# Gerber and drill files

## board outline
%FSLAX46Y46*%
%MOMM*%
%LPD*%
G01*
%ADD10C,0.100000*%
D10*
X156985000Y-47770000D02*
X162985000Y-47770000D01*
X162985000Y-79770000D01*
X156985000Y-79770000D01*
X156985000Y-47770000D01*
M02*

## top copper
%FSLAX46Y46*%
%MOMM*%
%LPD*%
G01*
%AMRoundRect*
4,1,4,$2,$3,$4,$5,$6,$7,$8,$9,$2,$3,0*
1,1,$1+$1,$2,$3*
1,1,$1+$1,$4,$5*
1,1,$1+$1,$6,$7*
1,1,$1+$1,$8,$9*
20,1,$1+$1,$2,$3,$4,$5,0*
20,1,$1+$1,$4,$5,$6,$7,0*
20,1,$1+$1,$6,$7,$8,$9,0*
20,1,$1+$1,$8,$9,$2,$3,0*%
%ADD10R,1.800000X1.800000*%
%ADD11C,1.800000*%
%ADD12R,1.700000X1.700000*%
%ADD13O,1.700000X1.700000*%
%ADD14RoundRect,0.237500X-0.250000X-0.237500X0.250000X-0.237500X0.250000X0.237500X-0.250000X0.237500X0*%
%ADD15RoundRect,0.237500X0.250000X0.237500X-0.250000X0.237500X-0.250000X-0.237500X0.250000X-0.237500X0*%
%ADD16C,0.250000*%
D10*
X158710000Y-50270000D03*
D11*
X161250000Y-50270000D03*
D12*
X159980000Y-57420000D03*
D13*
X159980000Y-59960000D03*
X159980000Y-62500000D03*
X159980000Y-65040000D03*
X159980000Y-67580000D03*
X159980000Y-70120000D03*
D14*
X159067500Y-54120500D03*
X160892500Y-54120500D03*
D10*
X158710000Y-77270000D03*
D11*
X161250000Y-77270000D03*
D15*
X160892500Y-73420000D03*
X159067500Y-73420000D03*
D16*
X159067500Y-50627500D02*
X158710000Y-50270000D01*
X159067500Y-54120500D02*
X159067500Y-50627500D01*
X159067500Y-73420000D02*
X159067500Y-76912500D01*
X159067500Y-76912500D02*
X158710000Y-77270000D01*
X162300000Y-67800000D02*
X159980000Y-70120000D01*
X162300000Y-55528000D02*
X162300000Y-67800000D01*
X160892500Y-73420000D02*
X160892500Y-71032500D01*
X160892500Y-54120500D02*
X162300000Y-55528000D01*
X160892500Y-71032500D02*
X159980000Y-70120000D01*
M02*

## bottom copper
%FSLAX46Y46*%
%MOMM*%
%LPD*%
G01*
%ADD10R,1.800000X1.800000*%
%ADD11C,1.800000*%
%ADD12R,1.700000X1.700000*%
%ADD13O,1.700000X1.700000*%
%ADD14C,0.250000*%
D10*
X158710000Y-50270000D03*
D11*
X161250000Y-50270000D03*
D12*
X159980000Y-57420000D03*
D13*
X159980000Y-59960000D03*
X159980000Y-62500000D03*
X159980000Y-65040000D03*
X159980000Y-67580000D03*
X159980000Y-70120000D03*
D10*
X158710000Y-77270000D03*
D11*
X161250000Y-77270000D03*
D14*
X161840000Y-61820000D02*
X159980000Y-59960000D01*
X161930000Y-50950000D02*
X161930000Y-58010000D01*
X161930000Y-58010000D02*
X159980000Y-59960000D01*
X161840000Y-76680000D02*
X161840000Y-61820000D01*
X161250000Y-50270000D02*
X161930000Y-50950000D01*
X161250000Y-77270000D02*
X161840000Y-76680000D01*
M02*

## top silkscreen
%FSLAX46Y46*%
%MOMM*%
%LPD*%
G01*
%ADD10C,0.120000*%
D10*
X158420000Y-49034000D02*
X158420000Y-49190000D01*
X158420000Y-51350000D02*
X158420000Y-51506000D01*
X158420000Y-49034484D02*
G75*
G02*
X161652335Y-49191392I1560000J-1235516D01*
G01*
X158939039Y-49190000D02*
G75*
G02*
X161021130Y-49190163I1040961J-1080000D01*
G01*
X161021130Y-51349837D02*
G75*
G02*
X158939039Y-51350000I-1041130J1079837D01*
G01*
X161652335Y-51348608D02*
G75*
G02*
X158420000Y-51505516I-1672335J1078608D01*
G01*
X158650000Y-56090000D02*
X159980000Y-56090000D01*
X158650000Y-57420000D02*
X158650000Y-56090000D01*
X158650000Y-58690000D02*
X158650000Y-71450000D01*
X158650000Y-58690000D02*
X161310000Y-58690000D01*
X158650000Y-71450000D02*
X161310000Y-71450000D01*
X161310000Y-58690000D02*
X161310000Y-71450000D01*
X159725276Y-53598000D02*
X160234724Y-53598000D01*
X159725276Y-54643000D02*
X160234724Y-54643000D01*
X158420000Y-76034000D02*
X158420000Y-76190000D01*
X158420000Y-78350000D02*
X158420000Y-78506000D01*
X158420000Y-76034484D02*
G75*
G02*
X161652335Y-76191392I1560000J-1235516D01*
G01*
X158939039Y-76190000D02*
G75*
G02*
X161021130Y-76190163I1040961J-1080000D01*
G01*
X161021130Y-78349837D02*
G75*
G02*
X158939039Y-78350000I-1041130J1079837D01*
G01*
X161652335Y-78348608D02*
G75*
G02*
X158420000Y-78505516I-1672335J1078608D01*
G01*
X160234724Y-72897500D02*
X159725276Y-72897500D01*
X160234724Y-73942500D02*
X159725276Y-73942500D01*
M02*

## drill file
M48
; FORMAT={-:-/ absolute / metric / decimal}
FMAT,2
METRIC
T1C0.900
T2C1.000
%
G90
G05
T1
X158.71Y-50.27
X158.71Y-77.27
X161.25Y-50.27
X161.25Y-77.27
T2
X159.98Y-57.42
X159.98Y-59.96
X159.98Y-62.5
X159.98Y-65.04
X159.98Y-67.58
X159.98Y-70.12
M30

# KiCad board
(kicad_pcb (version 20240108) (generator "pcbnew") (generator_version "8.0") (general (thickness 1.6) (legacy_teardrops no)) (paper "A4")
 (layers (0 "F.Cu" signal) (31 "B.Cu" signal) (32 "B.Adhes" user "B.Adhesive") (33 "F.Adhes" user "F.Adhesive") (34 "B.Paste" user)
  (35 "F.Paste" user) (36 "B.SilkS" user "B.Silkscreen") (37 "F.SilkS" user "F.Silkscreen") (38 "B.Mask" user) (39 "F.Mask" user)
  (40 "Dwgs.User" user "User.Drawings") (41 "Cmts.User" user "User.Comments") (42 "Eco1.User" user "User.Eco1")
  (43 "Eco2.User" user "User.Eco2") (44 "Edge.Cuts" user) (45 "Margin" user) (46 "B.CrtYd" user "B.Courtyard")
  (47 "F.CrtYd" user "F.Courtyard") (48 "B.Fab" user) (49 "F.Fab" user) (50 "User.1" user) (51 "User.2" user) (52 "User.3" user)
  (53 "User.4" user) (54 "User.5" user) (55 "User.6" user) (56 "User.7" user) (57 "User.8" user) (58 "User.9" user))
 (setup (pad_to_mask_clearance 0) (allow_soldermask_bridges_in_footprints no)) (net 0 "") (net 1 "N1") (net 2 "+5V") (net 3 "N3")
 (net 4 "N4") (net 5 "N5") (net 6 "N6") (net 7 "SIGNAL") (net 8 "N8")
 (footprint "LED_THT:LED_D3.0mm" (layer "F.Cu") (at 158.71 50.27)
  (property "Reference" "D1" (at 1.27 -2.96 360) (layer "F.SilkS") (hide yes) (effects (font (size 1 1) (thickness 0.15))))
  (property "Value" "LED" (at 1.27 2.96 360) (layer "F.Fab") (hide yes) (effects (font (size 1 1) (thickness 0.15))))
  (fp_line (start -0.29 -1.236) (end -0.29 -1.08) (stroke (width 0.12) (type solid)) (layer "F.SilkS"))
  (fp_line (start -0.29 1.08) (end -0.29 1.236) (stroke (width 0.12) (type solid)) (layer "F.SilkS"))
  (fp_arc (start -0.29 -1.235516) (mid 1.366487 -1.987659) (end 2.942335 -1.078608) (stroke (width 0.12) (type solid)) (layer "F.SilkS"))
  (fp_arc (start 0.229039 -1.08) (mid 1.270117 -1.5) (end 2.31113 -1.079837) (stroke (width 0.12) (type solid)) (layer "F.SilkS"))
  (fp_arc (start 2.31113 1.079837) (mid 1.270117 1.5) (end 0.229039 1.08) (stroke (width 0.12) (type solid)) (layer "F.SilkS"))
  (fp_arc (start 2.942335 1.078608) (mid 1.366487 1.987659) (end -0.29 1.235516) (stroke (width 0.12) (type solid)) (layer "F.SilkS"))
  (pad "1" thru_hole rect (at 0 0) (size 1.8 1.8) (drill 0.9) (layers "*.Cu" "*.Mask") (remove_unused_layers no) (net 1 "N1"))
  (pad "2" thru_hole circle (at 2.54 0) (size 1.8 1.8) (drill 0.9) (layers "*.Cu" "*.Mask") (remove_unused_layers no) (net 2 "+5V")))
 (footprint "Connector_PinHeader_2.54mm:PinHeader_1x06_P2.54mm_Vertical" (layer "F.Cu") (at 159.98 57.42)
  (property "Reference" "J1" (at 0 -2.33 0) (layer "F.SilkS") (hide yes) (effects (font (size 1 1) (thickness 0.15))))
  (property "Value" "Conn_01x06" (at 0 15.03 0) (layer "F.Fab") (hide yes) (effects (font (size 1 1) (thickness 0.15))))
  (fp_line (start -1.33 -1.33) (end 0 -1.33) (stroke (width 0.12) (type solid)) (layer "F.SilkS"))
  (fp_line (start -1.33 0) (end -1.33 -1.33) (stroke (width 0.12) (type solid)) (layer "F.SilkS"))
  (fp_line (start -1.33 1.27) (end -1.33 14.03) (stroke (width 0.12) (type solid)) (layer "F.SilkS"))
  (fp_line (start -1.33 1.27) (end 1.33 1.27) (stroke (width 0.12) (type solid)) (layer "F.SilkS"))
  (fp_line (start -1.33 14.03) (end 1.33 14.03) (stroke (width 0.12) (type solid)) (layer "F.SilkS"))
  (fp_line (start 1.33 1.27) (end 1.33 14.03) (stroke (width 0.12) (type solid)) (layer "F.SilkS"))
  (pad "1" thru_hole rect (at 0 0) (size 1.7 1.7) (drill 1) (layers "*.Cu" "*.Mask") (remove_unused_layers no) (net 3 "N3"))
  (pad "2" thru_hole oval (at 0 2.54) (size 1.7 1.7) (drill 1) (layers "*.Cu" "*.Mask") (remove_unused_layers no) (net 2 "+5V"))
  (pad "3" thru_hole oval (at 0 5.08) (size 1.7 1.7) (drill 1) (layers "*.Cu" "*.Mask") (remove_unused_layers no) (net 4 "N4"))
  (pad "4" thru_hole oval (at 0 7.62) (size 1.7 1.7) (drill 1) (layers "*.Cu" "*.Mask") (remove_unused_layers no) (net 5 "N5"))
  (pad "5" thru_hole oval (at 0 10.16) (size 1.7 1.7) (drill 1) (layers "*.Cu" "*.Mask") (remove_unused_layers no) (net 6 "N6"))
  (pad "6" thru_hole oval (at 0 12.7) (size 1.7 1.7) (drill 1) (layers "*.Cu" "*.Mask") (remove_unused_layers no) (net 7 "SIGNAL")))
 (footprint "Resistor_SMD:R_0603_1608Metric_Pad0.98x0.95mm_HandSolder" (layer "F.Cu") (at 159.98 54.1205)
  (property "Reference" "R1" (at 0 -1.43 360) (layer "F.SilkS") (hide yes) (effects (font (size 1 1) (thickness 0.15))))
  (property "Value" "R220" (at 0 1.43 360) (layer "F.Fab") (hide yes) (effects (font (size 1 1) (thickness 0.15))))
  (fp_line (start -0.254724 -0.5225) (end 0.254724 -0.5225) (stroke (width 0.12) (type solid)) (layer "F.SilkS"))
  (fp_line (start -0.254724 0.5225) (end 0.254724 0.5225) (stroke (width 0.12) (type solid)) (layer "F.SilkS"))
  (pad "1" smd roundrect (at -0.9125 0) (size 0.975 0.95) (layers "F.Cu" "F.Paste" "F.Mask") (roundrect_rratio 0.25) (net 1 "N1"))
  (pad "2" smd roundrect (at 0.9125 0) (size 0.975 0.95) (layers "F.Cu" "F.Paste" "F.Mask") (roundrect_rratio 0.25) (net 7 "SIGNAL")))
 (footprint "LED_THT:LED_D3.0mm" (layer "F.Cu") (at 158.71 77.27)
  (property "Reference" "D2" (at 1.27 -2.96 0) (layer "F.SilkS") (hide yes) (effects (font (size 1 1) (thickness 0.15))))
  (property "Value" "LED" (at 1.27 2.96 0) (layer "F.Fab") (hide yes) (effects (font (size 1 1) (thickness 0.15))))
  (fp_line (start -0.29 -1.236) (end -0.29 -1.08) (stroke (width 0.12) (type solid)) (layer "F.SilkS"))
  (fp_line (start -0.29 1.08) (end -0.29 1.236) (stroke (width 0.12) (type solid)) (layer "F.SilkS"))
  (fp_arc (start -0.29 -1.235516) (mid 1.366487 -1.987659) (end 2.942335 -1.078608) (stroke (width 0.12) (type solid)) (layer "F.SilkS"))
  (fp_arc (start 0.229039 -1.08) (mid 1.270117 -1.5) (end 2.31113 -1.079837) (stroke (width 0.12) (type solid)) (layer "F.SilkS"))
  (fp_arc (start 2.31113 1.079837) (mid 1.270117 1.5) (end 0.229039 1.08) (stroke (width 0.12) (type solid)) (layer "F.SilkS"))
  (fp_arc (start 2.942335 1.078608) (mid 1.366487 1.987659) (end -0.29 1.235516) (stroke (width 0.12) (type solid)) (layer "F.SilkS"))
  (pad "1" thru_hole rect (at 0 0) (size 1.8 1.8) (drill 0.9) (layers "*.Cu" "*.Mask") (remove_unused_layers no) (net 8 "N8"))
  (pad "2" thru_hole circle (at 2.54 0) (size 1.8 1.8) (drill 0.9) (layers "*.Cu" "*.Mask") (remove_unused_layers no) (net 2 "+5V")))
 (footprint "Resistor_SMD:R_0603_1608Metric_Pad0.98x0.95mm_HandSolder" (layer "F.Cu") (at 159.98 73.42 180)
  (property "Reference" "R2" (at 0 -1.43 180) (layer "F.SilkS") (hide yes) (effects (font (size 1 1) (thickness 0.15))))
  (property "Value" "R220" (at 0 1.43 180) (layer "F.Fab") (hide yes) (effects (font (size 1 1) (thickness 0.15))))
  (fp_line (start -0.254724 0.5225) (end 0.254724 0.5225) (stroke (width 0.12) (type solid)) (layer "F.SilkS"))
  (fp_line (start -0.254724 -0.5225) (end 0.254724 -0.5225) (stroke (width 0.12) (type solid)) (layer "F.SilkS"))
  (pad "1" smd roundrect (at -0.9125 0 180) (size 0.975 0.95) (layers "F.Cu" "F.Paste" "F.Mask") (roundrect_rratio 0.25) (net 7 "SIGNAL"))
  (pad "2" smd roundrect (at 0.9125 0 180) (size 0.975 0.95) (layers "F.Cu" "F.Paste" "F.Mask") (roundrect_rratio 0.25) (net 8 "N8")))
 (gr_rect (start 156.985 47.77) (end 162.985 79.77) (stroke (width 0.1) (type default)) (fill none) (layer "Edge.Cuts"))
 (segment (start 159.0675 50.6275) (end 158.71 50.27) (width 0.25) (layer "F.Cu") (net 1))
 (segment (start 159.0675 54.1205) (end 159.0675 50.6275) (width 0.25) (layer "F.Cu") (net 1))
 (segment (start 161.84 61.82) (end 159.98 59.96) (width 0.25) (layer "B.Cu") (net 2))
 (segment (start 161.93 50.95) (end 161.93 58.01) (width 0.25) (layer "B.Cu") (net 2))
 (segment (start 161.93 58.01) (end 159.98 59.96) (width 0.25) (layer "B.Cu") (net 2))
 (segment (start 161.84 76.68) (end 161.84 61.82) (width 0.25) (layer "B.Cu") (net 2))
 (segment (start 161.25 50.27) (end 161.93 50.95) (width 0.25) (layer "B.Cu") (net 2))
 (segment (start 161.25 77.27) (end 161.84 76.68) (width 0.25) (layer "B.Cu") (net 2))
 (segment (start 159.0675 73.42) (end 159.0675 76.9125) (width 0.25) (layer "F.Cu") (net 8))
 (segment (start 159.0675 76.9125) (end 158.71 77.27) (width 0.25) (layer "F.Cu") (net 8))
 (segment (start 162.3 67.8) (end 159.98 70.12) (width 0.25) (layer "F.Cu") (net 7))
 (segment (start 162.3 55.528) (end 162.3 67.8) (width 0.25) (layer "F.Cu") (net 7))
 (segment (start 160.8925 73.42) (end 160.8925 71.0325) (width 0.25) (layer "F.Cu") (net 7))
 (segment (start 160.8925 54.1205) (end 162.3 55.528) (width 0.25) (layer "F.Cu") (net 7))
 (segment (start 160.8925 71.0325) (end 159.98 70.12) (width 0.25) (layer "F.Cu") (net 7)))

